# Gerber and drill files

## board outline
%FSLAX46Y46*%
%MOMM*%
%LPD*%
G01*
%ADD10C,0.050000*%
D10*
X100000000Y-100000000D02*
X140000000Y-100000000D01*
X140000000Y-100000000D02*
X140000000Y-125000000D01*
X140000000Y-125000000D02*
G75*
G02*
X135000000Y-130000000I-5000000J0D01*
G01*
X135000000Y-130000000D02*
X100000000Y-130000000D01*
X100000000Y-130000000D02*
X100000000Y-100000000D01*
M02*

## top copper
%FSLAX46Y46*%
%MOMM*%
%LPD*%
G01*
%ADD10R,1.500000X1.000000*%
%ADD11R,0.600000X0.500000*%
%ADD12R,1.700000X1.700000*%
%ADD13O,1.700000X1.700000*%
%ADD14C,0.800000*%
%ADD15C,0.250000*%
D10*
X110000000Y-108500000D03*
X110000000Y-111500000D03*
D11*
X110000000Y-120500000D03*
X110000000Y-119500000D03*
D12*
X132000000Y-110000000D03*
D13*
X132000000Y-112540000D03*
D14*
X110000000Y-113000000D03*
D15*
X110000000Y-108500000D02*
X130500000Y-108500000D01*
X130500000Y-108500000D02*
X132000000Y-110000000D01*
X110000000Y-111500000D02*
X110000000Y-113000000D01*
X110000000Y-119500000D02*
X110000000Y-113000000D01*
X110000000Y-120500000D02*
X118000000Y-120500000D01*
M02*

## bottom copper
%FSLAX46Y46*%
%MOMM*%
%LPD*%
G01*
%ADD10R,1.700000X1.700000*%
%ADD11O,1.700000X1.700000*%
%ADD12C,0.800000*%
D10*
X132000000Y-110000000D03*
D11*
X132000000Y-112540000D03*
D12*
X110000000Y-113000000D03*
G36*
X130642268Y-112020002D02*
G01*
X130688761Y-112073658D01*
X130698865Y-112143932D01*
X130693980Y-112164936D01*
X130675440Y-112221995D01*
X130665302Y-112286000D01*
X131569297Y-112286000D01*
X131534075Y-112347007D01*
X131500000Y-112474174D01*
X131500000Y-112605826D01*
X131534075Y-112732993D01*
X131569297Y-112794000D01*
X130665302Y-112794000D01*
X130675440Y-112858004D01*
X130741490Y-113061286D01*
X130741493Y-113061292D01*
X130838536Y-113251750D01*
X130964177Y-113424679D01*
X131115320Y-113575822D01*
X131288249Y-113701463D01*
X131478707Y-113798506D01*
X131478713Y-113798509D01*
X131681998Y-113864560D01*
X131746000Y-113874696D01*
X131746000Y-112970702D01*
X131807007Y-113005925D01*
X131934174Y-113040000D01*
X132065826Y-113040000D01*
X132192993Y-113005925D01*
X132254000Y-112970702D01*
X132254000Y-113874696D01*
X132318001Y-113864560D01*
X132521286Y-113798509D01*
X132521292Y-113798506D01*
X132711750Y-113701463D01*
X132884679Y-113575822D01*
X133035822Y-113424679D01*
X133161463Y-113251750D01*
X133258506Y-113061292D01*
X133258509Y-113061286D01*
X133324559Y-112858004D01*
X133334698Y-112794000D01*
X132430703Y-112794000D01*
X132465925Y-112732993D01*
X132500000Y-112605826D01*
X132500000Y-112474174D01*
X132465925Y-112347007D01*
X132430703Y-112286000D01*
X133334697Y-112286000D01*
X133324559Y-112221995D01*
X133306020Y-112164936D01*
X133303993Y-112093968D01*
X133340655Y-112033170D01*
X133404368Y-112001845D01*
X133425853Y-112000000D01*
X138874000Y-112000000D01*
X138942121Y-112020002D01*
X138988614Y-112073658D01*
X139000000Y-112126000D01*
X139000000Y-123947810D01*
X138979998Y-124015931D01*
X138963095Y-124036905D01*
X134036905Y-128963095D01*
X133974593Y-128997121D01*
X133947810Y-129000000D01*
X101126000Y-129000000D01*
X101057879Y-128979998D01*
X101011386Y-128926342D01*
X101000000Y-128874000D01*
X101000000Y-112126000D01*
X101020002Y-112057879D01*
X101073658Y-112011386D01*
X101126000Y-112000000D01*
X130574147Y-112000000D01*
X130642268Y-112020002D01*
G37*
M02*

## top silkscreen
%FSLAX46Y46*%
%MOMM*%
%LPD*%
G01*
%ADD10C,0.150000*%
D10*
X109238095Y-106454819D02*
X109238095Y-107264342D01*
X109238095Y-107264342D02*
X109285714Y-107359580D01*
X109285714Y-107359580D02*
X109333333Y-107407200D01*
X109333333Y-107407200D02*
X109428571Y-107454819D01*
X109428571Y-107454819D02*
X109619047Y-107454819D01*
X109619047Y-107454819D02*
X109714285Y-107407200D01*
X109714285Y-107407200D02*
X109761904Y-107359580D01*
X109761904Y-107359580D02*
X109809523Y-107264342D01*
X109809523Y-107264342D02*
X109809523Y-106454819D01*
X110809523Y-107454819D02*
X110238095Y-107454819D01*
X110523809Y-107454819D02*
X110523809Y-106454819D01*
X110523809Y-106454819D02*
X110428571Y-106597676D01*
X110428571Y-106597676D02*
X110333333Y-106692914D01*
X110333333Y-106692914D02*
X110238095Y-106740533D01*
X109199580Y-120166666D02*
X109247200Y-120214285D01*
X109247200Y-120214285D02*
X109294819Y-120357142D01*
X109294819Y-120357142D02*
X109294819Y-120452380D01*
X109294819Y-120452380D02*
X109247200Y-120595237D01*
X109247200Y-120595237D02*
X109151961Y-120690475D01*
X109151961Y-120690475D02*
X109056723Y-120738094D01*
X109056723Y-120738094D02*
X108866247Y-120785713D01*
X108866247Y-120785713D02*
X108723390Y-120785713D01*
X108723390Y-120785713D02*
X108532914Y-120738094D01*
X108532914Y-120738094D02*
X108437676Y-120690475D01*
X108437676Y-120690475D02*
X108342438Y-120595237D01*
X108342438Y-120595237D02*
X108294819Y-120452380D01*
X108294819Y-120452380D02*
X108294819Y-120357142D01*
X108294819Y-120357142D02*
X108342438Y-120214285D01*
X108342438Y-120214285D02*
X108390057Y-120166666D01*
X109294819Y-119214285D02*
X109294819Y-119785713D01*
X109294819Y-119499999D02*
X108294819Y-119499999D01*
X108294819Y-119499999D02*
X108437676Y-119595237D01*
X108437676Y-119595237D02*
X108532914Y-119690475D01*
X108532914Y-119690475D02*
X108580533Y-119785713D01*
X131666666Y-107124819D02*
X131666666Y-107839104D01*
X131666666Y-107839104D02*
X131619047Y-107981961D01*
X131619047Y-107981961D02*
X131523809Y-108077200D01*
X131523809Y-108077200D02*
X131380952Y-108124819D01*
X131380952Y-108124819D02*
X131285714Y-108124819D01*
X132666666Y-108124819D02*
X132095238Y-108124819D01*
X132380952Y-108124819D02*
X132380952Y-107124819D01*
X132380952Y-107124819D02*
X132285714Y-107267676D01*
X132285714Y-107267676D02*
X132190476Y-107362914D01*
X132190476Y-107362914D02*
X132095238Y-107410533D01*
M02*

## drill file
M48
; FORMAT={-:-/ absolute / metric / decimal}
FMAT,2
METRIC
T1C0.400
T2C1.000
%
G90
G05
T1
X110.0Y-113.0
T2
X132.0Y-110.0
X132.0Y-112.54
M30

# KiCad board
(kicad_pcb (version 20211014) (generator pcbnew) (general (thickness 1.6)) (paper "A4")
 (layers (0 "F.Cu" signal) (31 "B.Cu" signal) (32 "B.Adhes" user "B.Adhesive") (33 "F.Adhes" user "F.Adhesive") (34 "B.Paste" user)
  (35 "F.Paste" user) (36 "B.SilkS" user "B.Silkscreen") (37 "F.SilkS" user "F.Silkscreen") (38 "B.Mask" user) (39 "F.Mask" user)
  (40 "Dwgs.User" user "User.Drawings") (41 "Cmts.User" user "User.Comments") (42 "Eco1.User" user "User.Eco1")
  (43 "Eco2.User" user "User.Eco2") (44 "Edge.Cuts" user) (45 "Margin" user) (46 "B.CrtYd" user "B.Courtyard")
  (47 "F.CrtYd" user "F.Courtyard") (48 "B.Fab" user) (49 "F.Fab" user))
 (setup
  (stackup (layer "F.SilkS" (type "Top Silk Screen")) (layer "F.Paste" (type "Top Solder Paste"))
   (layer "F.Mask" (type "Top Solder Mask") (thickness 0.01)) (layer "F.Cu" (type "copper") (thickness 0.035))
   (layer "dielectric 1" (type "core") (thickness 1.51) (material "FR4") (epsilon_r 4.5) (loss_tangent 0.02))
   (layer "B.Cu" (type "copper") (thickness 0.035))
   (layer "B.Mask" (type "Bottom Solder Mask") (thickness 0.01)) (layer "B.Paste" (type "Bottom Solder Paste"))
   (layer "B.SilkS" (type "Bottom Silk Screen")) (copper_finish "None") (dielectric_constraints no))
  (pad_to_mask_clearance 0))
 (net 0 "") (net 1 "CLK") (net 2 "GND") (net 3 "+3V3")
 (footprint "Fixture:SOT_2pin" (layer "F.Cu") (at 110 110)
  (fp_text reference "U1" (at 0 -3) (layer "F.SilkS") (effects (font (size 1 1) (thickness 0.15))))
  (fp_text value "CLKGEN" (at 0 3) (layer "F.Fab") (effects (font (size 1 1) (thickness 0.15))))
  (pad "1" smd rect (at 0 -1.5) (size 1.5 1) (layers "F.Cu" "F.Paste" "F.Mask") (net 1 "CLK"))
  (pad "2" smd rect (at 0 1.5) (size 1.5 1) (layers "F.Cu" "F.Paste" "F.Mask") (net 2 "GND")))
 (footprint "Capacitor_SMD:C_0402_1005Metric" (layer "F.Cu") (at 110 120 90)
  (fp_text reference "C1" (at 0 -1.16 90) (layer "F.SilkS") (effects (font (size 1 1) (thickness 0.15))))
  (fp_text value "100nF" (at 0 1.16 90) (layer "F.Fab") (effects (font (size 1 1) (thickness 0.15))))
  (pad "1" smd rect (at -0.5 0 90) (size 0.5 0.6) (layers "F.Cu" "F.Paste" "F.Mask") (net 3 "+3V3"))
  (pad "2" smd rect (at 0.5 0 90) (size 0.5 0.6) (layers "F.Cu" "F.Paste" "F.Mask") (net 2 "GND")))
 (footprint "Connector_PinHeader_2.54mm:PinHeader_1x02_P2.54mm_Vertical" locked (layer "F.Cu") (at 132 110)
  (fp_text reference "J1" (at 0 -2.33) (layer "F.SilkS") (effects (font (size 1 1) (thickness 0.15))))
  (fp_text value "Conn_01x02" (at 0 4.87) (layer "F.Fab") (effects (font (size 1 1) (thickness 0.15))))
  (pad "1" thru_hole rect (at 0 0) (size 1.7 1.7) (drill 1) (layers "*.Cu" "*.Mask") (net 1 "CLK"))
  (pad "2" thru_hole oval (at 0 2.54) (size 1.7 1.7) (drill 1) (layers "F&B.Cu" "*.Mask") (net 2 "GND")))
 (gr_line (start 100 100) (end 140 100) (width 0.05) (layer "Edge.Cuts"))
 (gr_line (start 140 100) (end 140 125) (width 0.05) (layer "Edge.Cuts"))
 (gr_arc (start 140 125) (mid 138.535534 128.535534) (end 135 130) (width 0.05) (layer "Edge.Cuts"))
 (gr_line (start 135 130) (end 100 130) (width 0.05) (layer "Edge.Cuts"))
 (gr_line (start 100 130) (end 100 100) (width 0.05) (layer "Edge.Cuts"))
 (segment (start 110 108.5) (end 130.5 108.5) (width 0.25) (layer "F.Cu") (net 1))
 (segment (start 130.5 108.5) (end 132 110) (width 0.25) (layer "F.Cu") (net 1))
 (segment (start 110 111.5) (end 110 113) (width 0.25) (layer "F.Cu") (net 2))
 (segment (start 110 119.5) (end 110 113) (width 0.25) (layer "F.Cu") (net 2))
 (segment (start 110 120.5) (end 118 120.5) (width 0.25) (layer "F.Cu") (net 3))
 (via (at 110 113) (size 0.8) (drill 0.4) (layers "F.Cu" "B.Cu") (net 2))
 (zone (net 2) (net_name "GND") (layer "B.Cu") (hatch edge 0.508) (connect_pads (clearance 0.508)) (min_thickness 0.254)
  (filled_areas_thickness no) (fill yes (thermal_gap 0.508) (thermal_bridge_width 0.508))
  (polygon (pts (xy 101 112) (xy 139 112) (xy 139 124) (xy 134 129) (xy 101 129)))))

